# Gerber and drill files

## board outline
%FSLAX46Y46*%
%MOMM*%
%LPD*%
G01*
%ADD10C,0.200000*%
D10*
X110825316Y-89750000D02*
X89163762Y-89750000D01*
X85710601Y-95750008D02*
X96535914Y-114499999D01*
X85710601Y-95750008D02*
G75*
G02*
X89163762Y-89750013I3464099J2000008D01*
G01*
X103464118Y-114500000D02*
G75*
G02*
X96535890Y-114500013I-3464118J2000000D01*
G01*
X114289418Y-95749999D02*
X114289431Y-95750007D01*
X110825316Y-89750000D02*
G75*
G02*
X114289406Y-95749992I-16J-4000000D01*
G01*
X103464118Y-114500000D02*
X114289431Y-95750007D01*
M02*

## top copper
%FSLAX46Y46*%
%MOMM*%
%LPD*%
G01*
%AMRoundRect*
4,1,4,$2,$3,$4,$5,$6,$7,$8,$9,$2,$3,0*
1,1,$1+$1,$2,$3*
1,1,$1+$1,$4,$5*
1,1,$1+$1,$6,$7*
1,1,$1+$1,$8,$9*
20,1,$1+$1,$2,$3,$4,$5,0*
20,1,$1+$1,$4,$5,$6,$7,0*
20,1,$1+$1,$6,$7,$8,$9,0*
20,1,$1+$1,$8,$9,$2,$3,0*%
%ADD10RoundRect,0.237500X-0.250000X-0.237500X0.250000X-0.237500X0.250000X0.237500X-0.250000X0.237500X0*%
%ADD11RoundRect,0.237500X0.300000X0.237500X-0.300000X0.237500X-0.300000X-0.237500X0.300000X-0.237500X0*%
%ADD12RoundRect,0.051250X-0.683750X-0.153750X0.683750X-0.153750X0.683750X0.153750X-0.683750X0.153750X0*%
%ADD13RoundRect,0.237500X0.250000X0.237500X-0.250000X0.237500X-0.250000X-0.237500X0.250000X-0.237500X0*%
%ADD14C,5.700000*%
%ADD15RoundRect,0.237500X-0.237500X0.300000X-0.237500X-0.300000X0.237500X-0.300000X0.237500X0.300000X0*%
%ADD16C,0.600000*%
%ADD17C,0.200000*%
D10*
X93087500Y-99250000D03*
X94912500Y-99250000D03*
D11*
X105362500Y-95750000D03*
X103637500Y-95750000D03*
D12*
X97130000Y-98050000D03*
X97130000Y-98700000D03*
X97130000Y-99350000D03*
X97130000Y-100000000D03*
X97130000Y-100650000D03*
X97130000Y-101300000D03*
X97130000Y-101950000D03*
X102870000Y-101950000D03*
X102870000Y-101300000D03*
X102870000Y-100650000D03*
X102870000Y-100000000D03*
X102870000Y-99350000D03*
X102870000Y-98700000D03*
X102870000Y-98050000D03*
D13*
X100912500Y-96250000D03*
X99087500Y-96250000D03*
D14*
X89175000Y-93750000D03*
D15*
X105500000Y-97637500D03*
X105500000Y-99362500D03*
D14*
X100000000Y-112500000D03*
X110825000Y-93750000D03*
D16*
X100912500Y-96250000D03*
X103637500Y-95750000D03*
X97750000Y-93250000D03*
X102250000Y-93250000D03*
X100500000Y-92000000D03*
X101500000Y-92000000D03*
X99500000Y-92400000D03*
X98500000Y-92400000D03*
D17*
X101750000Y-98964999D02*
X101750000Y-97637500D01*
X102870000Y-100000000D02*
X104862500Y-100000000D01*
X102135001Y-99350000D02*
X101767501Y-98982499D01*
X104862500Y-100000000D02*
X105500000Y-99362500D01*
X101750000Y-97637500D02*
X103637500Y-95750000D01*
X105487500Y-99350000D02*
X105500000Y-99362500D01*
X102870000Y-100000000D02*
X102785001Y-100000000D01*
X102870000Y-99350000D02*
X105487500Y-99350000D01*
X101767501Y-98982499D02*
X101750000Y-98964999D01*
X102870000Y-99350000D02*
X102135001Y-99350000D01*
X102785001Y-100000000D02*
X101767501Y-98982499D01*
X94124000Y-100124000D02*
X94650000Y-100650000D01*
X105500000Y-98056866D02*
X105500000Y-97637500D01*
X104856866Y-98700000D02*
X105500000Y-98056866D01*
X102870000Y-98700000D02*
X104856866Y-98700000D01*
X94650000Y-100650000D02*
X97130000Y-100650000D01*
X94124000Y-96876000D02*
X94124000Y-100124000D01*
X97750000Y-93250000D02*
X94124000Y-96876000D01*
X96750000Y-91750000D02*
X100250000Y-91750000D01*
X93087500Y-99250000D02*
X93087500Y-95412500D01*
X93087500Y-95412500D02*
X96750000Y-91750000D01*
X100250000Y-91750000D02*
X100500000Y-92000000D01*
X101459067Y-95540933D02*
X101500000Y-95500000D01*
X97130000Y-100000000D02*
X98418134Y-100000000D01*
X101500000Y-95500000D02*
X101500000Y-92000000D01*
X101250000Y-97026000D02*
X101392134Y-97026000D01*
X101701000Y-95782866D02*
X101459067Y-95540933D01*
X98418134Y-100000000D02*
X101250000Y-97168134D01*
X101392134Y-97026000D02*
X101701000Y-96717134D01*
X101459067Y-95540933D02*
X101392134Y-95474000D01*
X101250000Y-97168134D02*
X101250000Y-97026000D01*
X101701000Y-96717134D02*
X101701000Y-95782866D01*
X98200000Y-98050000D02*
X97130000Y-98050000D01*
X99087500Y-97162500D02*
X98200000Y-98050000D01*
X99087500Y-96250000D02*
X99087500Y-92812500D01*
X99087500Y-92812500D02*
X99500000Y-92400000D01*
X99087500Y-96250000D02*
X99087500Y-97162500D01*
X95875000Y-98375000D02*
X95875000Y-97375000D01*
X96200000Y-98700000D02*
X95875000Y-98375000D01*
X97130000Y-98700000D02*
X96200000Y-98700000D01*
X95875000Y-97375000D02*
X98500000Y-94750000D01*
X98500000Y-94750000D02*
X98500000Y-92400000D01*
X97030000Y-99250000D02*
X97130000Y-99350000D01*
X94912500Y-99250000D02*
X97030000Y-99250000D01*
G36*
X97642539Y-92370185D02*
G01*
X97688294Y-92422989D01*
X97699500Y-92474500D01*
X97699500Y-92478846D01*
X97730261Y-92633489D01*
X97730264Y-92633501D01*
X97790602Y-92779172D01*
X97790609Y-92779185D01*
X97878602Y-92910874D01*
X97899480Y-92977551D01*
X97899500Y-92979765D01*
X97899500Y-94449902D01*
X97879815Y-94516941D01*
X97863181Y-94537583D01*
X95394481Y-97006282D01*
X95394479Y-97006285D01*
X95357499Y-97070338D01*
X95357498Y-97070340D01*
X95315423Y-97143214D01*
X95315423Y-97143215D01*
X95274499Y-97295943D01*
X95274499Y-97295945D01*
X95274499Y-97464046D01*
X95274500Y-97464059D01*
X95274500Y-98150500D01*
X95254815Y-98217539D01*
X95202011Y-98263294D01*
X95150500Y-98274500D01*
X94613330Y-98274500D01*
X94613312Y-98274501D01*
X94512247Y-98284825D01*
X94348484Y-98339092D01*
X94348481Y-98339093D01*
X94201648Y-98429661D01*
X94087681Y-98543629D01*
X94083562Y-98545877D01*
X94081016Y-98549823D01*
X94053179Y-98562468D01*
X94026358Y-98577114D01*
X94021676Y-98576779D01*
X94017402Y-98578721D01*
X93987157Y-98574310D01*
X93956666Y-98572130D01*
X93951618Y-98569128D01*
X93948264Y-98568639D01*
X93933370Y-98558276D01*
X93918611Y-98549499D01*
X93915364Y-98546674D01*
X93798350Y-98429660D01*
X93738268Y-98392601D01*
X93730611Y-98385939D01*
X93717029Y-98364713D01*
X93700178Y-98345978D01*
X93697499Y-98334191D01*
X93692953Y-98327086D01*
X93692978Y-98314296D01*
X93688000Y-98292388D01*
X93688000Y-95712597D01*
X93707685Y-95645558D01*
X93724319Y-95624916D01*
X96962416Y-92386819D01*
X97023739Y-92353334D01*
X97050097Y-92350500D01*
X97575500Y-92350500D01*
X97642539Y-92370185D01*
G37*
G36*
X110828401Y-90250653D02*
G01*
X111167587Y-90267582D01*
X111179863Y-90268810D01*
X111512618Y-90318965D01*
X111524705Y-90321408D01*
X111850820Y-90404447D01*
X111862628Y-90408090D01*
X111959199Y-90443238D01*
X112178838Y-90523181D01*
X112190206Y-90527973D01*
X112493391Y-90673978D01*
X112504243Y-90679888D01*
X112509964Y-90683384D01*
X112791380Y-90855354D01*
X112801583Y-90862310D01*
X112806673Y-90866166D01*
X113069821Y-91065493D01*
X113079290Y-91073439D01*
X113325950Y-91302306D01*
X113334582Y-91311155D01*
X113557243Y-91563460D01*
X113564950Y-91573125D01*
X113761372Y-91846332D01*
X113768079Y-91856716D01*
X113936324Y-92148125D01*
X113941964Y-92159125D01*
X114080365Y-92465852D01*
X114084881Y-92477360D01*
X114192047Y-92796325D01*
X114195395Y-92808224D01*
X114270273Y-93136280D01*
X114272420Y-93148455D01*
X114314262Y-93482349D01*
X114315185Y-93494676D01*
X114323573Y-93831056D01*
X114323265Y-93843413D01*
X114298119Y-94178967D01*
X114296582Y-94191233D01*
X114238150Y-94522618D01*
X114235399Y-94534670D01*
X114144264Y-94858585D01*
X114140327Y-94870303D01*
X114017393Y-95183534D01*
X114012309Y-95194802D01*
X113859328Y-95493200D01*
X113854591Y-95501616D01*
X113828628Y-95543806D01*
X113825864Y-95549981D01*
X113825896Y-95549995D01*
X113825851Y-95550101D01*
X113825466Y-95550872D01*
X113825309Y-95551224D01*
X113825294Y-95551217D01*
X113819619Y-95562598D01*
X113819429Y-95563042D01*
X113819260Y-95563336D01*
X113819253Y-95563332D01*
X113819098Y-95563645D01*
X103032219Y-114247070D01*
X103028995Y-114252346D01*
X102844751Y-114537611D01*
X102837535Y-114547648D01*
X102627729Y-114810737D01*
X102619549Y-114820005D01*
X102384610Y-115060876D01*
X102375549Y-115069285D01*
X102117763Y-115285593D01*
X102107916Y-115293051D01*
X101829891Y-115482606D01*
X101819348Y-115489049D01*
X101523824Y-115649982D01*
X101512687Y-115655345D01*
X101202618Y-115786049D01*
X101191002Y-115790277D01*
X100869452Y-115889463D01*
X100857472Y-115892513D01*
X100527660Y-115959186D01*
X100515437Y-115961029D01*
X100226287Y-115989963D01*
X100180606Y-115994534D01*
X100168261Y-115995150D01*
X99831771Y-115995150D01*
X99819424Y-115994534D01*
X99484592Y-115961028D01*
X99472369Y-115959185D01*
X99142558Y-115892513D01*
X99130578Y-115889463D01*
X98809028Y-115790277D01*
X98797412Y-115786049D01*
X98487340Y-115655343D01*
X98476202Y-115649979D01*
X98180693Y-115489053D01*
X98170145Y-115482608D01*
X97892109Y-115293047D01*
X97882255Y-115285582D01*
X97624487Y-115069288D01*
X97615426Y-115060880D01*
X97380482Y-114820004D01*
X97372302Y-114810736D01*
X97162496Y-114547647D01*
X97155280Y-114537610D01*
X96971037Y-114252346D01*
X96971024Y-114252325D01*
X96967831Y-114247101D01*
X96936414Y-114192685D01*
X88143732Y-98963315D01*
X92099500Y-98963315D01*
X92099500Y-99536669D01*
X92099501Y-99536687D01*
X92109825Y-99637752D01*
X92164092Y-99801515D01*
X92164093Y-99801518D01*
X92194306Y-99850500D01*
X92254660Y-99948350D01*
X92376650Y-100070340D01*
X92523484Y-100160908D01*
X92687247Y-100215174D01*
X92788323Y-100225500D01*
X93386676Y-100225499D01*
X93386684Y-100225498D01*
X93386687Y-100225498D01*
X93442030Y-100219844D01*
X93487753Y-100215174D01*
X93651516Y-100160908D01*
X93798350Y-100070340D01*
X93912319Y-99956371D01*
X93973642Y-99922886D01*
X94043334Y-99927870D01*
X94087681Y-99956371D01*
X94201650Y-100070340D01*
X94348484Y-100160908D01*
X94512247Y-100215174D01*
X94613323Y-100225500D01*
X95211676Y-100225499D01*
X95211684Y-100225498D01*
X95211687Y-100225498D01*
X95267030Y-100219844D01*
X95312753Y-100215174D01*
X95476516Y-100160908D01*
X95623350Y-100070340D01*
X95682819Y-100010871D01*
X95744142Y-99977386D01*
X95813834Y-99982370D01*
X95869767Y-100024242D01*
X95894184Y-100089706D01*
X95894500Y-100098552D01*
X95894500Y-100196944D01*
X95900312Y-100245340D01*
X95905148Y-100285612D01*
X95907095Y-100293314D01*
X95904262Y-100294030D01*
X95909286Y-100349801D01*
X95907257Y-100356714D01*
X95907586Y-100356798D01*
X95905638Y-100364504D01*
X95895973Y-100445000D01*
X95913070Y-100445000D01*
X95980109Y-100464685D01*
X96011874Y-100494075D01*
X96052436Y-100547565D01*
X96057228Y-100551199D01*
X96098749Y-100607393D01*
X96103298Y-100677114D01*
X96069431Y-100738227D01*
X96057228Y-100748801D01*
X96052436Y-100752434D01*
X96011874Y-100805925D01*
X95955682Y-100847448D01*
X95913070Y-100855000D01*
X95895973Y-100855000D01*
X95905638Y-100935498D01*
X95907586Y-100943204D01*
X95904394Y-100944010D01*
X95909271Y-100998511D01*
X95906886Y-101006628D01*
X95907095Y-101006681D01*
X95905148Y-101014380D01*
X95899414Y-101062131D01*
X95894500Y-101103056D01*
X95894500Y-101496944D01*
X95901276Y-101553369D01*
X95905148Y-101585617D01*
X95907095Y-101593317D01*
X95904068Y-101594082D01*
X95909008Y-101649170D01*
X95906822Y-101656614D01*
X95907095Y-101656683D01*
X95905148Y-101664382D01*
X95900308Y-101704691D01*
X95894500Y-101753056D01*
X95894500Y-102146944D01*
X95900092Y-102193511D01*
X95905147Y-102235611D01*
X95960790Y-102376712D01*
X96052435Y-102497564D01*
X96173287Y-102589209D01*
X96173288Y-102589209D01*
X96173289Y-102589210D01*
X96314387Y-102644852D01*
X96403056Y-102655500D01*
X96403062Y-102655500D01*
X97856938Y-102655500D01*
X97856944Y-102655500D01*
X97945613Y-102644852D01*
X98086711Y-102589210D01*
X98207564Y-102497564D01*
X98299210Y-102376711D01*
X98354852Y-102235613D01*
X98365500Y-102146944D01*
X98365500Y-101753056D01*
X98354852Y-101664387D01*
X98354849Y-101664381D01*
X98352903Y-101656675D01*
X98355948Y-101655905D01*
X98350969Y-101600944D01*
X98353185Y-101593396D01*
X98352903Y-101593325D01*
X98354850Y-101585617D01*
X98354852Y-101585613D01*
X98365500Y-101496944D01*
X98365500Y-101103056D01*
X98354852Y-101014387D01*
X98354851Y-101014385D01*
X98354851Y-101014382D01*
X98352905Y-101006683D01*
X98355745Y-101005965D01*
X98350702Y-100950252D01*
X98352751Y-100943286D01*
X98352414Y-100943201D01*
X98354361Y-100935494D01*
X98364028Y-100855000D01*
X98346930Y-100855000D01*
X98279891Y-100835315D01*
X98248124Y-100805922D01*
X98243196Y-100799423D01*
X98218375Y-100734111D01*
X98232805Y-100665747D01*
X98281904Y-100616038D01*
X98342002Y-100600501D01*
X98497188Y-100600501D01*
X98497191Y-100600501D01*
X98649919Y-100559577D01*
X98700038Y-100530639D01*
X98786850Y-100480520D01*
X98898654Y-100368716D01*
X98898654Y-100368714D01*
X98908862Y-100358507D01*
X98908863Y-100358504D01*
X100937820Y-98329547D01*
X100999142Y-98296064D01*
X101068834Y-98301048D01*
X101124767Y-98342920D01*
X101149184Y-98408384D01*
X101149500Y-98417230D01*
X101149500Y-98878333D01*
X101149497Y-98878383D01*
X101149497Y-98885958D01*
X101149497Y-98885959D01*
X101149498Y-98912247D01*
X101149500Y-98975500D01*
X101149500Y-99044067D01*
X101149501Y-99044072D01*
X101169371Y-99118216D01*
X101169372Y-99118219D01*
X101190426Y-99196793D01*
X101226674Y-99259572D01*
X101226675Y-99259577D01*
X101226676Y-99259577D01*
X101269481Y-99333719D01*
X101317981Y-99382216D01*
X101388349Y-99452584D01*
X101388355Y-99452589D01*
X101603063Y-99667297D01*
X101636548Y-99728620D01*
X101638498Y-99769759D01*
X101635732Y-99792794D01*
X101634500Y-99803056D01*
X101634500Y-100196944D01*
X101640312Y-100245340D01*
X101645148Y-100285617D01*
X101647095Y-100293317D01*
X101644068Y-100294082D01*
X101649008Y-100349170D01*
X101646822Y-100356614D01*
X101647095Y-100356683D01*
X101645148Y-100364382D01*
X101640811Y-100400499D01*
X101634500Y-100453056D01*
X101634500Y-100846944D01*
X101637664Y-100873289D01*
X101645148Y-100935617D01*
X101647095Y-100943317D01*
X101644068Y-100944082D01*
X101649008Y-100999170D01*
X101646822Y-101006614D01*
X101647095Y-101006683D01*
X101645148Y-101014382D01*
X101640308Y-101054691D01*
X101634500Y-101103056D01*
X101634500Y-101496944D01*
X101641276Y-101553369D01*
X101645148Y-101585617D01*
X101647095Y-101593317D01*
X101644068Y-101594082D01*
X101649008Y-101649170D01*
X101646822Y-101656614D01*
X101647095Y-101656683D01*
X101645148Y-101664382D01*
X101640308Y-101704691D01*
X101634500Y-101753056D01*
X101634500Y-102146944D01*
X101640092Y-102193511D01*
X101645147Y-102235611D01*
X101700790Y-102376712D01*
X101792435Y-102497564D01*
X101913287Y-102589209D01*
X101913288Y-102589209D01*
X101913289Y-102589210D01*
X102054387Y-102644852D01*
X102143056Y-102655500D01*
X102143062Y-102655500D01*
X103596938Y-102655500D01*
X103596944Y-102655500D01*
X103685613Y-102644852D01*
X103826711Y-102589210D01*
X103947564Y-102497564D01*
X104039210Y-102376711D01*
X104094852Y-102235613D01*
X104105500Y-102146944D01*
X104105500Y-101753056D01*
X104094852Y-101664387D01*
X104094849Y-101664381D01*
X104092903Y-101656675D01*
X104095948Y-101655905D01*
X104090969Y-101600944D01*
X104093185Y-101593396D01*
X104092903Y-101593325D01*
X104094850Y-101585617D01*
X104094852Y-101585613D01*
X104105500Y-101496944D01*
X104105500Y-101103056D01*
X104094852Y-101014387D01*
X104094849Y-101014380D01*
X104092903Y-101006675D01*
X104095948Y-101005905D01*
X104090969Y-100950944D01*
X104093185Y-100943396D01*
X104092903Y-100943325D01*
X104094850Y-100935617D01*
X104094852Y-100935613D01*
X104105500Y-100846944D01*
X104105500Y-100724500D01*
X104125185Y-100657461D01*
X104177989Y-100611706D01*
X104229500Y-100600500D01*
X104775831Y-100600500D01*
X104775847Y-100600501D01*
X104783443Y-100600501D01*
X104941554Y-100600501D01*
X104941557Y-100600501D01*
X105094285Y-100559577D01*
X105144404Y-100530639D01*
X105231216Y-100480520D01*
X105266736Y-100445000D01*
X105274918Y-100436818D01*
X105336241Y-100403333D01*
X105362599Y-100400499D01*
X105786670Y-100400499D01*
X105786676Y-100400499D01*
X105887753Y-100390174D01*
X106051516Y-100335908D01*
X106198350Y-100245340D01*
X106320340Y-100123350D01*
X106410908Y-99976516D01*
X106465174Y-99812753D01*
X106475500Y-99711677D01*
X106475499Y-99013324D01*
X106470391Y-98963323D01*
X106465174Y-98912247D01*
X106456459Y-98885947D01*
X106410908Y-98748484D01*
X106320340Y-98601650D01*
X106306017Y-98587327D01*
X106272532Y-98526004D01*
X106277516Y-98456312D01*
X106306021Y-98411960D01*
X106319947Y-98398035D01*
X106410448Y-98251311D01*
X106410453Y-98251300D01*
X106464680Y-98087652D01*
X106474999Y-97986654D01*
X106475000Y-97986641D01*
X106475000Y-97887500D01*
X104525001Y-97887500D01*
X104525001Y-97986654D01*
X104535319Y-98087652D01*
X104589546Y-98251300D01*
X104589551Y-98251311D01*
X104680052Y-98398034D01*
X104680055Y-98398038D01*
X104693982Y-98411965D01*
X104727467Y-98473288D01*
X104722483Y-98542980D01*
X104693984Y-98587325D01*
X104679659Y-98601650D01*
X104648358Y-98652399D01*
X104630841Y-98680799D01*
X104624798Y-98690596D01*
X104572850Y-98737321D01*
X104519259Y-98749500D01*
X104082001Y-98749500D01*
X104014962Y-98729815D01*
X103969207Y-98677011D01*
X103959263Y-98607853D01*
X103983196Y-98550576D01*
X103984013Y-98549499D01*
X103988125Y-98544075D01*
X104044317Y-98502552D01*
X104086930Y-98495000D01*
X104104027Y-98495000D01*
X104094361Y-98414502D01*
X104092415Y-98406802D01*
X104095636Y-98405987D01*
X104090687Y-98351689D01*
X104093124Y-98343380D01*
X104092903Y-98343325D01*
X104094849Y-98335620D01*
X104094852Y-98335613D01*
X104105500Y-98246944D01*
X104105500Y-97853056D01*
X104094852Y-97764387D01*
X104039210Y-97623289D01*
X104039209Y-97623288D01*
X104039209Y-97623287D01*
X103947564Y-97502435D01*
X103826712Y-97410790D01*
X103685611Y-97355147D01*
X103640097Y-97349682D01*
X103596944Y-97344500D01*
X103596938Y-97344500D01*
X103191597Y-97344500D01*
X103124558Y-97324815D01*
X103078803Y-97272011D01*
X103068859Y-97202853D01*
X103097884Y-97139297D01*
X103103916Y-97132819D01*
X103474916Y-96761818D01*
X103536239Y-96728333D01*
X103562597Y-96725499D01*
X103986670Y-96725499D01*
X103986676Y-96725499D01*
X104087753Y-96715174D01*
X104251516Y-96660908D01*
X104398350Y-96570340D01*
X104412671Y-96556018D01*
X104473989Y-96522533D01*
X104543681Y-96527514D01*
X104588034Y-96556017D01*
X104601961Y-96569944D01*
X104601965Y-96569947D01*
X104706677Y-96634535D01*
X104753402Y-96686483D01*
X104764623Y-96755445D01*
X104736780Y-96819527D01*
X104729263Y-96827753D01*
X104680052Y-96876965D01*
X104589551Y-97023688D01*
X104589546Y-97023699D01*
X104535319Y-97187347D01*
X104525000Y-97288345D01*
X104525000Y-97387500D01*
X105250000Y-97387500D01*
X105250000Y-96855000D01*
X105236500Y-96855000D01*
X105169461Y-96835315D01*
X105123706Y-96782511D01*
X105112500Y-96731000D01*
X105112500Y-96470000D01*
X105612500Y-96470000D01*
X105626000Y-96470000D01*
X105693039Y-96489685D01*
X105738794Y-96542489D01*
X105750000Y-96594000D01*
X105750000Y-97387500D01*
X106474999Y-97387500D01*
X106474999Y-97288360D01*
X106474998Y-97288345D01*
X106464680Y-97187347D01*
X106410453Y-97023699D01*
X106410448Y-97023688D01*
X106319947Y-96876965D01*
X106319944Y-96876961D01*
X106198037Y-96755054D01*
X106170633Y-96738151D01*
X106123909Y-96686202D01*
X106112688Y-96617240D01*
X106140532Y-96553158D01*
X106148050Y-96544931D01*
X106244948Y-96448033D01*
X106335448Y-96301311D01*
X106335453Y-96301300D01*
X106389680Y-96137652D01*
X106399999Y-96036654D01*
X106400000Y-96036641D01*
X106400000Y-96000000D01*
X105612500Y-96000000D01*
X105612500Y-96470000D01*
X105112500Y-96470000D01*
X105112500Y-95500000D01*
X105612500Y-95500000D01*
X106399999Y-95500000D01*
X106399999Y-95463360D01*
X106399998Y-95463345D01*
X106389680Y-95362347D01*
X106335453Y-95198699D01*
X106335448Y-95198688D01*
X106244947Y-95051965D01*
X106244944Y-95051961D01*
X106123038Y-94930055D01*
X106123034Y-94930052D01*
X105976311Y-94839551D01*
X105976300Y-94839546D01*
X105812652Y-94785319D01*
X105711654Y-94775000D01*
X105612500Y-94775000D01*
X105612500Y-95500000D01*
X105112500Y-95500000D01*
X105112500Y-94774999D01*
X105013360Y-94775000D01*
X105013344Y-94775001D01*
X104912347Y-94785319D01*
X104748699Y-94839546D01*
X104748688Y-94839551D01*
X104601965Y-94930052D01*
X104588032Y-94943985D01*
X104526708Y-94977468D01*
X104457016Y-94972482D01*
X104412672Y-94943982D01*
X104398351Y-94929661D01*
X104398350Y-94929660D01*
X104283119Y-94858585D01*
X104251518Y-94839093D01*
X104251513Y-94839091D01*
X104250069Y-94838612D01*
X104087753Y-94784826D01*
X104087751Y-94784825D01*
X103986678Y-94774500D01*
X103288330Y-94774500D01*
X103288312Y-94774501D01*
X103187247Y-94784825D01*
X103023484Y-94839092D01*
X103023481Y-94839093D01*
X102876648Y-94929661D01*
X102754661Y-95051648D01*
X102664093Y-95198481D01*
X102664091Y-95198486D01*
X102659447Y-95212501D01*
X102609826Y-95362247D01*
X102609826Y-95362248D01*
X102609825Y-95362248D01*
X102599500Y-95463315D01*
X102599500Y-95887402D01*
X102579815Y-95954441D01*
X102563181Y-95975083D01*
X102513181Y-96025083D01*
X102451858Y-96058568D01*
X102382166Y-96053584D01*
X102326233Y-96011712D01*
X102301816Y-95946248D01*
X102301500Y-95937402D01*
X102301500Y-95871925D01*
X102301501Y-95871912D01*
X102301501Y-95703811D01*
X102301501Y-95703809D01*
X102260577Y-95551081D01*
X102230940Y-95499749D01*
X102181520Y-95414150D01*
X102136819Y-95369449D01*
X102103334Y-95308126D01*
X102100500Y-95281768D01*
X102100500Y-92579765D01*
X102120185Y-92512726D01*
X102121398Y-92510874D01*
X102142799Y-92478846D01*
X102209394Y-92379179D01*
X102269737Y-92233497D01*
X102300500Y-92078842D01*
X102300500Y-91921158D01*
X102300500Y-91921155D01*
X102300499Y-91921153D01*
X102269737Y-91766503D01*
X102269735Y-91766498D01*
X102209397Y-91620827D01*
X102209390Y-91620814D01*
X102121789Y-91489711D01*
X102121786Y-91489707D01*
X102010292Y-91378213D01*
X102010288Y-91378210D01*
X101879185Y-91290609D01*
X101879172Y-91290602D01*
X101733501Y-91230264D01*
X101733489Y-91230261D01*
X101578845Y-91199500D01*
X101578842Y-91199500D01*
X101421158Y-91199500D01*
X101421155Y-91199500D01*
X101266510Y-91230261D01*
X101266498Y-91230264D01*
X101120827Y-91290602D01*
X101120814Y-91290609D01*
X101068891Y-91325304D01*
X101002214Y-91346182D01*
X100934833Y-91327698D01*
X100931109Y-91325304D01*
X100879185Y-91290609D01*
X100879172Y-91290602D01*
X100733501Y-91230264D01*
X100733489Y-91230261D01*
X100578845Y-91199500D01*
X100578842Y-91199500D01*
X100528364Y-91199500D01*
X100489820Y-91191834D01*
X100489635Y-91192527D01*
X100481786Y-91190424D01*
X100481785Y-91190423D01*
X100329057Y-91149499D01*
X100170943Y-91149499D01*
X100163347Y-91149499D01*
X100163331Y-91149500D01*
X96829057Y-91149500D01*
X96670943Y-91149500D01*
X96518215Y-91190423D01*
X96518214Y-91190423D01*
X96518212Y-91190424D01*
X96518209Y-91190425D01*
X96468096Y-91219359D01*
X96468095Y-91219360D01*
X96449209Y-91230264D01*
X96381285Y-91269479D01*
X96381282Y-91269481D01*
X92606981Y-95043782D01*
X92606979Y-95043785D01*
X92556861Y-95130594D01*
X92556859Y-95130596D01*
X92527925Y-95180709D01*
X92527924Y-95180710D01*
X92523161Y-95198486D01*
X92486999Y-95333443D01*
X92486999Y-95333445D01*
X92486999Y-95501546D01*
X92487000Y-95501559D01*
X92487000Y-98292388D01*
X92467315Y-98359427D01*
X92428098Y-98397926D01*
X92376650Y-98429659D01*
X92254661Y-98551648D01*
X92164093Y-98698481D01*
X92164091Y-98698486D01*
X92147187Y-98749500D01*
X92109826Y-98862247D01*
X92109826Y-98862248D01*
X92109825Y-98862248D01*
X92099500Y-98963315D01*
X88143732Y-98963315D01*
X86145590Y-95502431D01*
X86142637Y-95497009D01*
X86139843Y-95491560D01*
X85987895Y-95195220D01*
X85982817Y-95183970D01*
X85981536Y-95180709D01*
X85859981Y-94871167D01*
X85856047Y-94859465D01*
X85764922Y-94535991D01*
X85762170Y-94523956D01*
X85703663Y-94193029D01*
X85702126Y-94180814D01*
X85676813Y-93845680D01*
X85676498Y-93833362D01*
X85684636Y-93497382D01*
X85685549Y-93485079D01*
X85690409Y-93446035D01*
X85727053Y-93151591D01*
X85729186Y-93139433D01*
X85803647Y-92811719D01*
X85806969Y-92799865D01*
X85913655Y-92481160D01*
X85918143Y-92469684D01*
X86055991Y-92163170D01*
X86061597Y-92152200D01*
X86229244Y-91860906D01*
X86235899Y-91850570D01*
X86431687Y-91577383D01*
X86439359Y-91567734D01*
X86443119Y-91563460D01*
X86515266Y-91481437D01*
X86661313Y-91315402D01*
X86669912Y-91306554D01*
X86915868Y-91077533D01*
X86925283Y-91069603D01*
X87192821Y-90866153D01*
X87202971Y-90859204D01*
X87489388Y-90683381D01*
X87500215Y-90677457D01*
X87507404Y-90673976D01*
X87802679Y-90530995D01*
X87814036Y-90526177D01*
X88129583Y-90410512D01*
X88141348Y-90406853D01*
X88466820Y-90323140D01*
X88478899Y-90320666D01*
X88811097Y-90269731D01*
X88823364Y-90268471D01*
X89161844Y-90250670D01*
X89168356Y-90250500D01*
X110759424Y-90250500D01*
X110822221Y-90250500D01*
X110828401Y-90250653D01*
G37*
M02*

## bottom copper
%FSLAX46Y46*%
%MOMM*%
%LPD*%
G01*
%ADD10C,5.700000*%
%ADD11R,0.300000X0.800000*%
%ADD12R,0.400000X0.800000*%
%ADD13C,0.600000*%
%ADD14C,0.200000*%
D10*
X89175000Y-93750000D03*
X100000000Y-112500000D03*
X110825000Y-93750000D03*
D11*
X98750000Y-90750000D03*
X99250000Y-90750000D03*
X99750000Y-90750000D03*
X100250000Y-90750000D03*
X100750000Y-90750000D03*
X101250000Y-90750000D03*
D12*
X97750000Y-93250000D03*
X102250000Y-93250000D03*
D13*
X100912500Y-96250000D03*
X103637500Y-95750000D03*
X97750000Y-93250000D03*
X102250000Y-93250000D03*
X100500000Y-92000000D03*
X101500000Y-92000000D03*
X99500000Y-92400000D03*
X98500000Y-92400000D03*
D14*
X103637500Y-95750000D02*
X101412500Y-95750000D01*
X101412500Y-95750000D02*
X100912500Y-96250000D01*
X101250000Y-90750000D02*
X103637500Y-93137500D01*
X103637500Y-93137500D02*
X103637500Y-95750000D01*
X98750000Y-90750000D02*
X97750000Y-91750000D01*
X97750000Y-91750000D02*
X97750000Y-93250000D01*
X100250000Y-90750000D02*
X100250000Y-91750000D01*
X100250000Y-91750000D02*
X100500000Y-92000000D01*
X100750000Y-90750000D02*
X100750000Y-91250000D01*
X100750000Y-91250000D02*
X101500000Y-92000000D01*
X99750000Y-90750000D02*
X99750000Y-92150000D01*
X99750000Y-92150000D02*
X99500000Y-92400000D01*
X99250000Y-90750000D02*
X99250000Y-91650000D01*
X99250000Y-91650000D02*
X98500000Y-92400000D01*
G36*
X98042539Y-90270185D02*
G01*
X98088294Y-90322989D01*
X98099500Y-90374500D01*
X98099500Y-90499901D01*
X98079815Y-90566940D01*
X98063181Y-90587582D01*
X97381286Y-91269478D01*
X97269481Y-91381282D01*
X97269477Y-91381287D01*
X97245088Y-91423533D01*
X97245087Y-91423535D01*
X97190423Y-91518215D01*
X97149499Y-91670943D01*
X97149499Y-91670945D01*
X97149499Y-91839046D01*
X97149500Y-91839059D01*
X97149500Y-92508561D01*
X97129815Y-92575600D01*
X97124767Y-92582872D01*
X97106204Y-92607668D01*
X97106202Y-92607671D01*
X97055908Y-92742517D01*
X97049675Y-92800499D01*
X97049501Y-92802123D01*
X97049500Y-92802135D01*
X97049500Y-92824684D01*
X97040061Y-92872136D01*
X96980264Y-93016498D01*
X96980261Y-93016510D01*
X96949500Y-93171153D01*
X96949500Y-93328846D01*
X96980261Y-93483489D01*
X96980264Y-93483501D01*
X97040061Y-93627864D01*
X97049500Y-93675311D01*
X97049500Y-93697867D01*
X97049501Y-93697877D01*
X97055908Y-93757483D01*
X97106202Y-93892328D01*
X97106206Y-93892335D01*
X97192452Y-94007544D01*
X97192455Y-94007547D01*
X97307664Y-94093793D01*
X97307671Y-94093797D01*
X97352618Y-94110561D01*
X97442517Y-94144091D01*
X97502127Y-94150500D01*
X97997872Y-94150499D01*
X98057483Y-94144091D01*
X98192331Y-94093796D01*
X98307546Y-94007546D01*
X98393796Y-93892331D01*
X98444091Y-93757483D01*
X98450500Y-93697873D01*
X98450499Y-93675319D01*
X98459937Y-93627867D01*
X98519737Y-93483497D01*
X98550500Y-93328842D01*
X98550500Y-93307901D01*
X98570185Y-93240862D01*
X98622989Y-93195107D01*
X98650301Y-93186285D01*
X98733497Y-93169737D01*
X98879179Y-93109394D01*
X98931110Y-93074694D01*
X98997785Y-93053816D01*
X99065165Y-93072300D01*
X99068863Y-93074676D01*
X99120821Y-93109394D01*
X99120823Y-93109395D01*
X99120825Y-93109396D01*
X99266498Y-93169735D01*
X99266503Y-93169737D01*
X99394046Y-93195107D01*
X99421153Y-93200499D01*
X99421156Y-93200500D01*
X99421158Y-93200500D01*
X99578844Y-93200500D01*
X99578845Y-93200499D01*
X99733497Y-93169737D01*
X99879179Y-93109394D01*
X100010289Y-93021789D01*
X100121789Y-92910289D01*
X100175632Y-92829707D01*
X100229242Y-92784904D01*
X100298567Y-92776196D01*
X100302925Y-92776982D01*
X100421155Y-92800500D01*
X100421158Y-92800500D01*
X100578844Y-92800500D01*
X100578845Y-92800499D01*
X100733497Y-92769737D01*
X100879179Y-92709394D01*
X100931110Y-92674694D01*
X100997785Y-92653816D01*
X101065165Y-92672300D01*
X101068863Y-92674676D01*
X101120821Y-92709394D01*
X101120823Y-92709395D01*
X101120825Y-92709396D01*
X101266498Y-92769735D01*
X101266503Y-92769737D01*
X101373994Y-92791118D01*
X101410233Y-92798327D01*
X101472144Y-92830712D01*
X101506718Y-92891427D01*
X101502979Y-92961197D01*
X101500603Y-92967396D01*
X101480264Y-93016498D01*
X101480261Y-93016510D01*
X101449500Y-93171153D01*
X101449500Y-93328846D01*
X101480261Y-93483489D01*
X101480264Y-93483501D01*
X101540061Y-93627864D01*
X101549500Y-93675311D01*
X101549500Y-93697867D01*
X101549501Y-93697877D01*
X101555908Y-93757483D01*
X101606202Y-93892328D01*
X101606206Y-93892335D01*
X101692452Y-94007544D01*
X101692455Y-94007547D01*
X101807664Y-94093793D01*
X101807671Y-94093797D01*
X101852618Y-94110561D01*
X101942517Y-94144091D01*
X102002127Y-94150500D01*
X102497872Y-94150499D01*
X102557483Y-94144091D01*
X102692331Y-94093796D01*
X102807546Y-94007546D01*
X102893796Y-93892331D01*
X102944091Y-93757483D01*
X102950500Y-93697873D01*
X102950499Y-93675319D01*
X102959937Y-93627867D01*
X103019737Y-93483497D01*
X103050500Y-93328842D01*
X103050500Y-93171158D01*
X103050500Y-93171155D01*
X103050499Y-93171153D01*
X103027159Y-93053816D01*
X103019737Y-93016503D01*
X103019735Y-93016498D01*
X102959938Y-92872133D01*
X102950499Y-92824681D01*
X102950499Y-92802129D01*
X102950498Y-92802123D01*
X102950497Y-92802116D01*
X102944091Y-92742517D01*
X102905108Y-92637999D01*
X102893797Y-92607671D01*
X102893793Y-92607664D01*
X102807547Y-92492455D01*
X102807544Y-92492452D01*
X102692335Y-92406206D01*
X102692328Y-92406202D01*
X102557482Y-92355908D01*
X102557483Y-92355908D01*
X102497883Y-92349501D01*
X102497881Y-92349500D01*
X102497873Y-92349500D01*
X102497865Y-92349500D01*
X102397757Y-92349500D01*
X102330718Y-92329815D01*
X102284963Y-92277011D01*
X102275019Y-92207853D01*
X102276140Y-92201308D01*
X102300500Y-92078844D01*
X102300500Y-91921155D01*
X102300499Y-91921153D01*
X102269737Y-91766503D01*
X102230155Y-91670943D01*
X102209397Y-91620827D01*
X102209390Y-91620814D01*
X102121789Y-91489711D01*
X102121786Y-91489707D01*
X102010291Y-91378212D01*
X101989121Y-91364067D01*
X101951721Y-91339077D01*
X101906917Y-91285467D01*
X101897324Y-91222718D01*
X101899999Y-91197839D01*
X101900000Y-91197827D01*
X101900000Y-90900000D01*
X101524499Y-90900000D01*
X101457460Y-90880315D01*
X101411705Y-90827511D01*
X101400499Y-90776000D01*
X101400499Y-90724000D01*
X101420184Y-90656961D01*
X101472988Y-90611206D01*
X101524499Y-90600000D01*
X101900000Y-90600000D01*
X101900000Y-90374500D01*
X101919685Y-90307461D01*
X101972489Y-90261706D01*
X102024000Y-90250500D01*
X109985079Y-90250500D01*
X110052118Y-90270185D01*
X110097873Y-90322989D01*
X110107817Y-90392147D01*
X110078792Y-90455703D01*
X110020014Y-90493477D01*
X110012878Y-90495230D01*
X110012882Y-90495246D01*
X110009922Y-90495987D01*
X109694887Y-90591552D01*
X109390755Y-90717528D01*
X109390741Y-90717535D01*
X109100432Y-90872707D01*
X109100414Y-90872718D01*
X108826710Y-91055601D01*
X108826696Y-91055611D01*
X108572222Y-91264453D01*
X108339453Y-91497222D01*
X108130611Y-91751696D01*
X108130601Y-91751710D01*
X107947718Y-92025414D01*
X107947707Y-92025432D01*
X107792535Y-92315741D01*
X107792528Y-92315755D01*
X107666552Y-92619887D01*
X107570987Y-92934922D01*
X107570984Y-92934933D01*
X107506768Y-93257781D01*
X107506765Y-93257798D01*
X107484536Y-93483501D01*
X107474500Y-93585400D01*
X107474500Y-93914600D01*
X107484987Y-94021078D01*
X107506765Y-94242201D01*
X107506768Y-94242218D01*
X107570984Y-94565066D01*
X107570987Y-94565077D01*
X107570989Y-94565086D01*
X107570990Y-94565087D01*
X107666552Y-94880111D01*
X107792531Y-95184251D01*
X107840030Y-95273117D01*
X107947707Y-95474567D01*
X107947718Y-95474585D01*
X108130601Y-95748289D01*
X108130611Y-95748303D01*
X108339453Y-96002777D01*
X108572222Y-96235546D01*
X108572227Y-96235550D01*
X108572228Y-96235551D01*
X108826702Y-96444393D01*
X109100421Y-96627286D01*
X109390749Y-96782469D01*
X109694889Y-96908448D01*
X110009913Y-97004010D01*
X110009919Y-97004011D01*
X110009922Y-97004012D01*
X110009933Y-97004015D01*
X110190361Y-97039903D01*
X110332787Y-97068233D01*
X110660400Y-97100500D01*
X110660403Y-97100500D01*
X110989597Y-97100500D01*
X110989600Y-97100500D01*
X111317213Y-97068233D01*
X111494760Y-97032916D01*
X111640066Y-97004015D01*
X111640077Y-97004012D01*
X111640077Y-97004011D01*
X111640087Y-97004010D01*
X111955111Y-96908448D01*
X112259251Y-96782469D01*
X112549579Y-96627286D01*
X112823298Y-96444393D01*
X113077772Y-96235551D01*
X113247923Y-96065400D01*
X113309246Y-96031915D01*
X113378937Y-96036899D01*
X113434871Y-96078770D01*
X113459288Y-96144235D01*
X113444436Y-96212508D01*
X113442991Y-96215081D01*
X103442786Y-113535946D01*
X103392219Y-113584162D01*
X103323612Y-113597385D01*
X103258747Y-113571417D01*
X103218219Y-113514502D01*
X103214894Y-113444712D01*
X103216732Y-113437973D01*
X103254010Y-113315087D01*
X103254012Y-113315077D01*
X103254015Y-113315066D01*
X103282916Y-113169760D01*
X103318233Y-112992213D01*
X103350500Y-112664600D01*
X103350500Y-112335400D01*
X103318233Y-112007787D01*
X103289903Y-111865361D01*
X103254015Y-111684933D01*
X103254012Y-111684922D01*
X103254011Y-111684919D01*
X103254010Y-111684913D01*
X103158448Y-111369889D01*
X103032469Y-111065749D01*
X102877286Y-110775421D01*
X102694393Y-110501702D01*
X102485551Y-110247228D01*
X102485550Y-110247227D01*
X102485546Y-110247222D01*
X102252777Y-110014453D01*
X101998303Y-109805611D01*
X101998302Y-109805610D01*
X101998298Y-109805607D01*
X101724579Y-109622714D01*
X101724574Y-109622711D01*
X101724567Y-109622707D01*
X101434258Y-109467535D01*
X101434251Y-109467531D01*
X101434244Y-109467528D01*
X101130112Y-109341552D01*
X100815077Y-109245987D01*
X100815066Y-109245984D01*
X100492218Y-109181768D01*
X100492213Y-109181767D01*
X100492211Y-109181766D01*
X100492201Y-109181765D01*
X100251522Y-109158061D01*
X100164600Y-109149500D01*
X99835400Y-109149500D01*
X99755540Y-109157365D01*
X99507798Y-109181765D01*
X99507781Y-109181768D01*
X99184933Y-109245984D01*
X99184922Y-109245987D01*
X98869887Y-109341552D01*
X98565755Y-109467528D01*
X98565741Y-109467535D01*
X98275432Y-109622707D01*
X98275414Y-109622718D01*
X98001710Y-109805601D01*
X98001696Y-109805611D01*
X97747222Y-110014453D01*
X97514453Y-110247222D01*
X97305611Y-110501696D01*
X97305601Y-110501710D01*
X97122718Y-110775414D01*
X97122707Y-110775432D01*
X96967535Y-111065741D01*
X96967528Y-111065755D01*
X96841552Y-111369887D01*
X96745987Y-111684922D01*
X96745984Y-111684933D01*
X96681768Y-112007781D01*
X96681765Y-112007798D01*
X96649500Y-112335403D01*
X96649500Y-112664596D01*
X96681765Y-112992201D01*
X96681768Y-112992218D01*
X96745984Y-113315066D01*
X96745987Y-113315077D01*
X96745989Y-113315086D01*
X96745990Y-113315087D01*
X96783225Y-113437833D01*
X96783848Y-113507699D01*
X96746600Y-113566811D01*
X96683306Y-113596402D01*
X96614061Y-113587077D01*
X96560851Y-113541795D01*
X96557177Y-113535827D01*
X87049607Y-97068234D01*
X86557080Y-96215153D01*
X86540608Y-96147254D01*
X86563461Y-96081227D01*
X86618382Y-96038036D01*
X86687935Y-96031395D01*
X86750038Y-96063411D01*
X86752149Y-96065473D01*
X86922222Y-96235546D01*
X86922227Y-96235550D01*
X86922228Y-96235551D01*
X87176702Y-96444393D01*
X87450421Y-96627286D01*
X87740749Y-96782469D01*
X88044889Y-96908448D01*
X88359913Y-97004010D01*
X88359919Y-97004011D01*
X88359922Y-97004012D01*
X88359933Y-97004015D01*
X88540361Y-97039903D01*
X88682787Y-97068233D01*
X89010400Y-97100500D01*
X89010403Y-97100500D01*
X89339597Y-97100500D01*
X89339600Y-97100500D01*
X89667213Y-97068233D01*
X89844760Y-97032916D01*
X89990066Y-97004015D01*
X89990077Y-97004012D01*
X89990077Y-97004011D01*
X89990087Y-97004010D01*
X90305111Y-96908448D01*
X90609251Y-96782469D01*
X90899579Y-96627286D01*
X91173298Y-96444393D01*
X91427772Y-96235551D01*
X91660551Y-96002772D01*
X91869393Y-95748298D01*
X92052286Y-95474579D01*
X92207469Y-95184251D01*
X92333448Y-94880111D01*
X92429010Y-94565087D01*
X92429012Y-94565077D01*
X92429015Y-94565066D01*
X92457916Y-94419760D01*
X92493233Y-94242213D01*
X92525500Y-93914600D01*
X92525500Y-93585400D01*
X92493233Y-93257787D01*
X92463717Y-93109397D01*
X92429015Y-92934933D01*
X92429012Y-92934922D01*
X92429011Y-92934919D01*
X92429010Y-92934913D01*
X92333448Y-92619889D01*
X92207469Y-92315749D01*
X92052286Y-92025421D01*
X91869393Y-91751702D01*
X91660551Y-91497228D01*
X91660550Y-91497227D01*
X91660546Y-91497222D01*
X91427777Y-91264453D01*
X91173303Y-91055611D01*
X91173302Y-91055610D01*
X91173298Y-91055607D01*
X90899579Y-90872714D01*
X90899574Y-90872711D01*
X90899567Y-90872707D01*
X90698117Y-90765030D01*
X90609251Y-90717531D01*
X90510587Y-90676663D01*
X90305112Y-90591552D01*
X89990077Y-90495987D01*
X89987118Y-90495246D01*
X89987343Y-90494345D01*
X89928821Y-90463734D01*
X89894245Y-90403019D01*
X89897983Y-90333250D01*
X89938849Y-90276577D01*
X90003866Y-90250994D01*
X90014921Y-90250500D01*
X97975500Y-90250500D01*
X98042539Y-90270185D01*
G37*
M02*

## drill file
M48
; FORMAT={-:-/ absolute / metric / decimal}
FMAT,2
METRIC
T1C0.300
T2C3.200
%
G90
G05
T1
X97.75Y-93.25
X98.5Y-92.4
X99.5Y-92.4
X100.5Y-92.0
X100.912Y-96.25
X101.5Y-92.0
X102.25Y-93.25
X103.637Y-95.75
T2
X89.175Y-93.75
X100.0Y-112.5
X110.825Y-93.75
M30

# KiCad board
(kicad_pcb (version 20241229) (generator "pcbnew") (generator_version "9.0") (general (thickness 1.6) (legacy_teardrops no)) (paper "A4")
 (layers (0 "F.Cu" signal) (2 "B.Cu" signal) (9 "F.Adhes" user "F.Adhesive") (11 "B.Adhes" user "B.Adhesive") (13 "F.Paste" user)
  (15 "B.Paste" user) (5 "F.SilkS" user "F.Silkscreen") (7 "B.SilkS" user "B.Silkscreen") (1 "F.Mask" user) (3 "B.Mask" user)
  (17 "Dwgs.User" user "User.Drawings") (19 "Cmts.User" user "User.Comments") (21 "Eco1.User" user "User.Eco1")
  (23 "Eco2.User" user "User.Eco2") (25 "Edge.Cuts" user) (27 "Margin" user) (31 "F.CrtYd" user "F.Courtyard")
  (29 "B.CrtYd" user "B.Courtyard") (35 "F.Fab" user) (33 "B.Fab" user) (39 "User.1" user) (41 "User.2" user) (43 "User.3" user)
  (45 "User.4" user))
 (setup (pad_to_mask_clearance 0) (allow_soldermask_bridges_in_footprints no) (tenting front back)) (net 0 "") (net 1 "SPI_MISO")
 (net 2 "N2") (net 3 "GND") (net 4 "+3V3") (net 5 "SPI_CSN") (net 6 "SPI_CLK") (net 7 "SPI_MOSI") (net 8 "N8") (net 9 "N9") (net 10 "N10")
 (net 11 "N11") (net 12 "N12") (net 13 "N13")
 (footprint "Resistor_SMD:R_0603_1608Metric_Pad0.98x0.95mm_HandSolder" (layer "F.Cu") (at 94 99.25)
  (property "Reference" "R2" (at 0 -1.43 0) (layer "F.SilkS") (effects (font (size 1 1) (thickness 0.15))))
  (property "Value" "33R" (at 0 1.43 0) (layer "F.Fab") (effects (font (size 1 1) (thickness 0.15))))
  (pad "1" smd roundrect (at -0.9125 0) (size 0.975 0.95) (layers "F.Cu" "F.Mask" "F.Paste") (roundrect_rratio 0.25) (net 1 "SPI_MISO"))
  (pad "2" smd roundrect (at 0.9125 0) (size 0.975 0.95) (layers "F.Cu" "F.Mask" "F.Paste") (roundrect_rratio 0.25) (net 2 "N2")))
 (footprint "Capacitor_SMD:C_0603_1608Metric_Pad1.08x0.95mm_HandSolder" (layer "F.Cu") (at 104.5 95.75 180)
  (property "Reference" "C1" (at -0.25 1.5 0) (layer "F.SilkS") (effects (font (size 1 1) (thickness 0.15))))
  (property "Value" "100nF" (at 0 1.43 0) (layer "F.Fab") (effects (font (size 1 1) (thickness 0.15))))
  (pad "1" smd roundrect (at -0.8625 0 180) (size 1.075 0.95) (layers "F.Cu" "F.Mask" "F.Paste") (roundrect_rratio 0.25) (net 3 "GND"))
  (pad "2" smd roundrect (at 0.8625 0 180) (size 1.075 0.95) (layers "F.Cu" "F.Mask" "F.Paste") (roundrect_rratio 0.25) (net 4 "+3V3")))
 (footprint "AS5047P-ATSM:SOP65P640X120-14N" (layer "F.Cu") (at 100 100)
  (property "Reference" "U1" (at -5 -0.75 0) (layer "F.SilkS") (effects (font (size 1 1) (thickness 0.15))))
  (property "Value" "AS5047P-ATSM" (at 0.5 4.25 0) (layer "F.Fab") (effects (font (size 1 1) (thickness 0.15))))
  (pad "1" smd roundrect (at -2.87 -1.95) (size 1.47 0.41) (layers "F.Cu" "F.Mask" "F.Paste") (roundrect_rratio 0.125) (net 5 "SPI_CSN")
   (solder_mask_margin 0.102))
  (pad "2" smd roundrect (at -2.87 -1.3) (size 1.47 0.41) (layers "F.Cu" "F.Mask" "F.Paste") (roundrect_rratio 0.125) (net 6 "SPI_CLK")
   (solder_mask_margin 0.102))
  (pad "3" smd roundrect (at -2.87 -0.65) (size 1.47 0.41) (layers "F.Cu" "F.Mask" "F.Paste") (roundrect_rratio 0.125) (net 2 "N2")
   (solder_mask_margin 0.102))
  (pad "4" smd roundrect (at -2.87 0) (size 1.47 0.41) (layers "F.Cu" "F.Mask" "F.Paste") (roundrect_rratio 0.125) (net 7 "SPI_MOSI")
   (solder_mask_margin 0.102))
  (pad "5" smd roundrect (at -2.87 0.65) (size 1.47 0.41) (layers "F.Cu" "F.Mask" "F.Paste") (roundrect_rratio 0.125) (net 3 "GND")
   (solder_mask_margin 0.102))
  (pad "6" smd roundrect (at -2.87 1.3) (size 1.47 0.41) (layers "F.Cu" "F.Mask" "F.Paste") (roundrect_rratio 0.125) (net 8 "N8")
   (solder_mask_margin 0.102))
  (pad "7" smd roundrect (at -2.87 1.95) (size 1.47 0.41) (layers "F.Cu" "F.Mask" "F.Paste") (roundrect_rratio 0.125) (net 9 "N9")
   (solder_mask_margin 0.102))
  (pad "8" smd roundrect (at 2.87 1.95) (size 1.47 0.41) (layers "F.Cu" "F.Mask" "F.Paste") (roundrect_rratio 0.125) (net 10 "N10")
   (solder_mask_margin 0.102))
  (pad "9" smd roundrect (at 2.87 1.3) (size 1.47 0.41) (layers "F.Cu" "F.Mask" "F.Paste") (roundrect_rratio 0.125) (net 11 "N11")
   (solder_mask_margin 0.102))
  (pad "10" smd roundrect (at 2.87 0.65) (size 1.47 0.41) (layers "F.Cu" "F.Mask" "F.Paste") (roundrect_rratio 0.125) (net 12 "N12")
   (solder_mask_margin 0.102))
  (pad "11" smd roundrect (at 2.87 0) (size 1.47 0.41) (layers "F.Cu" "F.Mask" "F.Paste") (roundrect_rratio 0.125) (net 4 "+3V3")
   (solder_mask_margin 0.102))
  (pad "12" smd roundrect (at 2.87 -0.65) (size 1.47 0.41) (layers "F.Cu" "F.Mask" "F.Paste") (roundrect_rratio 0.125) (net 4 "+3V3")
   (solder_mask_margin 0.102))
  (pad "13" smd roundrect (at 2.87 -1.3) (size 1.47 0.41) (layers "F.Cu" "F.Mask" "F.Paste") (roundrect_rratio 0.125) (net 3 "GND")
   (solder_mask_margin 0.102))
  (pad "14" smd roundrect (at 2.87 -1.95) (size 1.47 0.41) (layers "F.Cu" "F.Mask" "F.Paste") (roundrect_rratio 0.125) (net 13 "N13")
   (solder_mask_margin 0.102)))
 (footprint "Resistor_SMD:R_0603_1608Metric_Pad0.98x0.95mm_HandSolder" (layer "F.Cu") (at 100 96.25 180)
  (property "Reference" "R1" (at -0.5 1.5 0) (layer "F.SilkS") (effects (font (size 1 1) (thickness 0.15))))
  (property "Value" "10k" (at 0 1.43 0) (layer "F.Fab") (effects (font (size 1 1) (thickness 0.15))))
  (pad "1" smd roundrect (at -0.9125 0 180) (size 0.975 0.95) (layers "F.Cu" "F.Mask" "F.Paste") (roundrect_rratio 0.25) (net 4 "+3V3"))
  (pad "2" smd roundrect (at 0.9125 0 180) (size 0.975 0.95) (layers "F.Cu" "F.Mask" "F.Paste") (roundrect_rratio 0.25) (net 5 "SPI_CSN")))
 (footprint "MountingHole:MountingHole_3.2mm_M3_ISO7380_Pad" (layer "F.Cu") (at 89.175 93.75)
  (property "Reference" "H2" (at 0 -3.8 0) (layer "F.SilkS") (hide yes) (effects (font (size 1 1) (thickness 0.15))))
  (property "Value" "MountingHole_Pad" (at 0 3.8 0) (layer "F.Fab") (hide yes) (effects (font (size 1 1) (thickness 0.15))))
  (pad "1" thru_hole circle (at 0 0) (size 5.7 5.7) (drill 3.2) (layers "*.Cu" "*.Mask") (remove_unused_layers no) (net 3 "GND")
   (zone_connect 2)))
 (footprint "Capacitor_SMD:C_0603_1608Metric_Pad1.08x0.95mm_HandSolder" (layer "F.Cu") (at 105.5 98.5 -90)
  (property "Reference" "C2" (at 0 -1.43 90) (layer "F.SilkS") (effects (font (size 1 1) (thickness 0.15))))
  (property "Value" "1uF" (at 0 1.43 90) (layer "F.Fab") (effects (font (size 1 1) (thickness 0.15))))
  (pad "1" smd roundrect (at -0.8625 0 270) (size 1.075 0.95) (layers "F.Cu" "F.Mask" "F.Paste") (roundrect_rratio 0.25) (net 3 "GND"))
  (pad "2" smd roundrect (at 0.8625 0 270) (size 1.075 0.95) (layers "F.Cu" "F.Mask" "F.Paste") (roundrect_rratio 0.25) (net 4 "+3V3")))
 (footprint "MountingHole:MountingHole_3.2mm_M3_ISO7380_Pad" (layer "F.Cu") (at 100 112.5)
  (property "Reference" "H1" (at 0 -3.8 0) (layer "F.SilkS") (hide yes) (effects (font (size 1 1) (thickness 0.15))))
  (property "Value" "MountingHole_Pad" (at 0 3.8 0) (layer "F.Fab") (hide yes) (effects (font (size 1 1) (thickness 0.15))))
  (pad "1" thru_hole circle (at 0 0) (size 5.7 5.7) (drill 3.2) (layers "*.Cu" "*.Mask") (remove_unused_layers no) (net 3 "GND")
   (zone_connect 2)))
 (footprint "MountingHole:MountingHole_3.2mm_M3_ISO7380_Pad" (layer "F.Cu") (at 110.825 93.75)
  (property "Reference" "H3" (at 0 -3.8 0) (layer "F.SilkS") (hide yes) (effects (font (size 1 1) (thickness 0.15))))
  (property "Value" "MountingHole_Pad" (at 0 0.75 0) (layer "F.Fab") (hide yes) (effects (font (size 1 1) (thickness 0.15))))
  (pad "1" thru_hole circle (at 0 0) (size 5.7 5.7) (drill 3.2) (layers "*.Cu" "*.Mask") (remove_unused_layers no) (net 3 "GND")
   (zone_connect 2)))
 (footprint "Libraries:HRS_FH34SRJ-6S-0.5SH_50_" (layer "B.Cu") (at 100 92 180)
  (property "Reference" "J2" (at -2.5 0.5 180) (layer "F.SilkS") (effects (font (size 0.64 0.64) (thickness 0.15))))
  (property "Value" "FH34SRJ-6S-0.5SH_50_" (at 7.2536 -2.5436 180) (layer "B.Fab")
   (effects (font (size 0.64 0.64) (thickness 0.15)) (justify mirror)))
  (pad "1" smd rect (at 1.25 1.25 180) (size 0.3 0.8) (layers "B.Cu" "B.Mask") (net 3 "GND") (solder_mask_margin 0.102))
  (pad "2" smd rect (at 0.75 1.25 180) (size 0.3 0.8) (layers "B.Cu" "B.Mask") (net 6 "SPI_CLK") (solder_mask_margin 0.102))
  (pad "3" smd rect (at 0.25 1.25 180) (size 0.3 0.8) (layers "B.Cu" "B.Mask") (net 5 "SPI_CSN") (solder_mask_margin 0.102))
  (pad "4" smd rect (at -0.25 1.25 180) (size 0.3 0.8) (layers "B.Cu" "B.Mask") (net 1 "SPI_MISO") (solder_mask_margin 0.102))
  (pad "5" smd rect (at -0.75 1.25 180) (size 0.3 0.8) (layers "B.Cu" "B.Mask") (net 7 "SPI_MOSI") (solder_mask_margin 0.102))
  (pad "6" smd rect (at -1.25 1.25 180) (size 0.3 0.8) (layers "B.Cu" "B.Mask") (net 4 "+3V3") (solder_mask_margin 0.102))
  (pad "S1" smd rect (at 2.25 -1.25 180) (size 0.4 0.8) (layers "B.Cu" "B.Mask" "B.Paste") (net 3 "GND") (solder_mask_margin 0.102))
  (pad "S2" smd rect (at -2.25 -1.25 180) (size 0.4 0.8) (layers "B.Cu" "B.Mask" "B.Paste") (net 3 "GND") (solder_mask_margin 0.102)))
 (gr_line (start 110.825316 89.75) (end 89.163762 89.75) (stroke (width 0.2) (type default)) (layer "Edge.Cuts"))
 (gr_line (start 85.710601 95.750008) (end 96.535914 114.499999) (stroke (width 0.2) (type default)) (layer "Edge.Cuts"))
 (gr_arc (start 85.710601 95.750008) (mid 85.710599 91.749997) (end 89.163762 89.75) (stroke (width 0.2) (type default)) (layer "Edge.Cuts"))
 (gr_arc (start 103.464118 114.5) (mid 100.000016 116.5) (end 96.535914 114.499999) (stroke (width 0.2) (type default)) (layer "Edge.Cuts"))
 (gr_line (start 114.289418 95.749999) (end 114.289431 95.750007) (stroke (width 0.2) (type default)) (layer "Edge.Cuts"))
 (gr_arc (start 110.825316 89.75) (mid 114.28942 91.750004) (end 114.289418 95.749999) (stroke (width 0.2) (type default))
  (layer "Edge.Cuts"))
 (gr_line (start 103.464118 114.5) (end 114.289431 95.750007) (stroke (width 0.2) (type default)) (layer "Edge.Cuts"))
 (segment (start 101.75 98.964999) (end 101.75 97.6375) (width 0.2) (layer "F.Cu") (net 4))
 (segment (start 102.87 100) (end 104.8625 100) (width 0.2) (layer "F.Cu") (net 4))
 (segment (start 102.135001 99.35) (end 101.767501 98.982499) (width 0.2) (layer "F.Cu") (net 4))
 (segment (start 104.8625 100) (end 105.5 99.3625) (width 0.2) (layer "F.Cu") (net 4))
 (segment (start 101.75 97.6375) (end 103.6375 95.75) (width 0.2) (layer "F.Cu") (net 4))
 (segment (start 105.4875 99.35) (end 105.5 99.3625) (width 0.2) (layer "F.Cu") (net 4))
 (segment (start 102.87 100) (end 102.785001 100) (width 0.2) (layer "F.Cu") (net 4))
 (segment (start 102.87 99.35) (end 105.4875 99.35) (width 0.2) (layer "F.Cu") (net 4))
 (segment (start 101.767501 98.982499) (end 101.75 98.964999) (width 0.2) (layer "F.Cu") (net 4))
 (segment (start 102.87 99.35) (end 102.135001 99.35) (width 0.2) (layer "F.Cu") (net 4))
 (segment (start 102.785001 100) (end 101.767501 98.982499) (width 0.2) (layer "F.Cu") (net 4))
 (via (at 100.9125 96.25) (size 0.6) (drill 0.3) (layers "F.Cu" "B.Cu") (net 4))
 (via (at 103.6375 95.75) (size 0.6) (drill 0.3) (layers "F.Cu" "B.Cu") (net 4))
 (segment (start 103.6375 95.75) (end 101.4125 95.75) (width 0.2) (layer "B.Cu") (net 4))
 (segment (start 101.4125 95.75) (end 100.9125 96.25) (width 0.2) (layer "B.Cu") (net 4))
 (segment (start 101.25 90.75) (end 103.6375 93.1375) (width 0.2) (layer "B.Cu") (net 4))
 (segment (start 103.6375 93.1375) (end 103.6375 95.75) (width 0.2) (layer "B.Cu") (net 4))
 (segment (start 94.124 100.124) (end 94.65 100.65) (width 0.2) (layer "F.Cu") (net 3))
 (segment (start 105.5 98.056866) (end 105.5 97.6375) (width 0.2) (layer "F.Cu") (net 3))
 (segment (start 104.856866 98.7) (end 105.5 98.056866) (width 0.2) (layer "F.Cu") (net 3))
 (segment (start 102.87 98.7) (end 104.856866 98.7) (width 0.2) (layer "F.Cu") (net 3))
 (segment (start 94.65 100.65) (end 97.13 100.65) (width 0.2) (layer "F.Cu") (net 3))
 (segment (start 94.124 96.876) (end 94.124 100.124) (width 0.2) (layer "F.Cu") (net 3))
 (segment (start 97.75 93.25) (end 94.124 96.876) (width 0.2) (layer "F.Cu") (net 3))
 (via (at 97.75 93.25) (size 0.6) (drill 0.3) (layers "F.Cu" "B.Cu") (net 3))
 (via (at 102.25 93.25) (size 0.6) (drill 0.3) (layers "F.Cu" "B.Cu") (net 3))
 (segment (start 98.75 90.75) (end 97.75 91.75) (width 0.2) (layer "B.Cu") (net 3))
 (segment (start 97.75 91.75) (end 97.75 93.25) (width 0.2) (layer "B.Cu") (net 3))
 (segment (start 96.75 91.75) (end 100.25 91.75) (width 0.2) (layer "F.Cu") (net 1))
 (segment (start 93.0875 99.25) (end 93.0875 95.4125) (width 0.2) (layer "F.Cu") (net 1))
 (segment (start 93.0875 95.4125) (end 96.75 91.75) (width 0.2) (layer "F.Cu") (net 1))
 (segment (start 100.25 91.75) (end 100.5 92) (width 0.2) (layer "F.Cu") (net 1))
 (via (at 100.5 92) (size 0.6) (drill 0.3) (layers "F.Cu" "B.Cu") (free yes) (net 1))
 (segment (start 100.25 90.75) (end 100.25 91.75) (width 0.2) (layer "B.Cu") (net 1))
 (segment (start 100.25 91.75) (end 100.5 92) (width 0.2) (layer "B.Cu") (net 1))
 (segment (start 101.459067 95.540933) (end 101.5 95.5) (width 0.2) (layer "F.Cu") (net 7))
 (segment (start 97.13 100) (end 98.418134 100) (width 0.2) (layer "F.Cu") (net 7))
 (segment (start 101.5 95.5) (end 101.5 92) (width 0.2) (layer "F.Cu") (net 7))
 (segment (start 101.25 97.026) (end 101.392134 97.026) (width 0.2) (layer "F.Cu") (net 7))
 (segment (start 101.701 95.782866) (end 101.459067 95.540933) (width 0.2) (layer "F.Cu") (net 7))
 (segment (start 98.418134 100) (end 101.25 97.168134) (width 0.2) (layer "F.Cu") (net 7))
 (segment (start 101.392134 97.026) (end 101.701 96.717134) (width 0.2) (layer "F.Cu") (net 7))
 (segment (start 101.459067 95.540933) (end 101.392134 95.474) (width 0.2) (layer "F.Cu") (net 7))
 (segment (start 101.25 97.168134) (end 101.25 97.026) (width 0.2) (layer "F.Cu") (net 7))
 (segment (start 101.701 96.717134) (end 101.701 95.782866) (width 0.2) (layer "F.Cu") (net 7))
 (via (at 101.5 92) (size 0.6) (drill 0.3) (layers "F.Cu" "B.Cu") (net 7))
 (segment (start 100.75 90.75) (end 100.75 91.25) (width 0.2) (layer "B.Cu") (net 7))
 (segment (start 100.75 91.25) (end 101.5 92) (width 0.2) (layer "B.Cu") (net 7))
 (segment (start 98.2 98.05) (end 97.13 98.05) (width 0.2) (layer "F.Cu") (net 5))
 (segment (start 99.0875 97.1625) (end 98.2 98.05) (width 0.2) (layer "F.Cu") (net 5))
 (segment (start 99.0875 96.25) (end 99.0875 92.8125) (width 0.2) (layer "F.Cu") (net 5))
 (segment (start 99.0875 92.8125) (end 99.5 92.4) (width 0.2) (layer "F.Cu") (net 5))
 (segment (start 99.0875 96.25) (end 99.0875 97.1625) (width 0.2) (layer "F.Cu") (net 5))
 (via (at 99.5 92.4) (size 0.6) (drill 0.3) (layers "F.Cu" "B.Cu") (free yes) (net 5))
 (segment (start 99.75 90.75) (end 99.75 92.15) (width 0.2) (layer "B.Cu") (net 5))
 (segment (start 99.75 92.15) (end 99.5 92.4) (width 0.2) (layer "B.Cu") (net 5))
 (segment (start 95.875 98.375) (end 95.875 97.375) (width 0.2) (layer "F.Cu") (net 6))
 (segment (start 96.2 98.7) (end 95.875 98.375) (width 0.2) (layer "F.Cu") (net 6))
 (segment (start 97.13 98.7) (end 96.2 98.7) (width 0.2) (layer "F.Cu") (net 6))
 (segment (start 95.875 97.375) (end 98.5 94.75) (width 0.2) (layer "F.Cu") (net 6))
 (segment (start 98.5 94.75) (end 98.5 92.4) (width 0.2) (layer "F.Cu") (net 6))
 (via (at 98.5 92.4) (size 0.6) (drill 0.3) (layers "F.Cu" "B.Cu") (free yes) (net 6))
 (segment (start 99.25 90.75) (end 99.25 91.65) (width 0.2) (layer "B.Cu") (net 6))
 (segment (start 99.25 91.65) (end 98.5 92.4) (width 0.2) (layer "B.Cu") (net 6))
 (segment (start 97.03 99.25) (end 97.13 99.35) (width 0.2) (layer "F.Cu") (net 2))
 (segment (start 94.9125 99.25) (end 97.03 99.25) (width 0.2) (layer "F.Cu") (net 2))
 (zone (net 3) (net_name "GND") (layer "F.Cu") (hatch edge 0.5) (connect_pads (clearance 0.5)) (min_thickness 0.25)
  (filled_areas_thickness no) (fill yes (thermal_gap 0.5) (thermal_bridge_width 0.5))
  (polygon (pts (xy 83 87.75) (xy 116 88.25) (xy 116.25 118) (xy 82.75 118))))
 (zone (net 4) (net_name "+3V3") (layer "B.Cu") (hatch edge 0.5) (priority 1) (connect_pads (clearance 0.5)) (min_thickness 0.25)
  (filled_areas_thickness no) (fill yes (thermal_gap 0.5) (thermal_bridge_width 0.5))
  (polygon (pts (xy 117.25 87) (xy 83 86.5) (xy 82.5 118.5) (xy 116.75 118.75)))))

